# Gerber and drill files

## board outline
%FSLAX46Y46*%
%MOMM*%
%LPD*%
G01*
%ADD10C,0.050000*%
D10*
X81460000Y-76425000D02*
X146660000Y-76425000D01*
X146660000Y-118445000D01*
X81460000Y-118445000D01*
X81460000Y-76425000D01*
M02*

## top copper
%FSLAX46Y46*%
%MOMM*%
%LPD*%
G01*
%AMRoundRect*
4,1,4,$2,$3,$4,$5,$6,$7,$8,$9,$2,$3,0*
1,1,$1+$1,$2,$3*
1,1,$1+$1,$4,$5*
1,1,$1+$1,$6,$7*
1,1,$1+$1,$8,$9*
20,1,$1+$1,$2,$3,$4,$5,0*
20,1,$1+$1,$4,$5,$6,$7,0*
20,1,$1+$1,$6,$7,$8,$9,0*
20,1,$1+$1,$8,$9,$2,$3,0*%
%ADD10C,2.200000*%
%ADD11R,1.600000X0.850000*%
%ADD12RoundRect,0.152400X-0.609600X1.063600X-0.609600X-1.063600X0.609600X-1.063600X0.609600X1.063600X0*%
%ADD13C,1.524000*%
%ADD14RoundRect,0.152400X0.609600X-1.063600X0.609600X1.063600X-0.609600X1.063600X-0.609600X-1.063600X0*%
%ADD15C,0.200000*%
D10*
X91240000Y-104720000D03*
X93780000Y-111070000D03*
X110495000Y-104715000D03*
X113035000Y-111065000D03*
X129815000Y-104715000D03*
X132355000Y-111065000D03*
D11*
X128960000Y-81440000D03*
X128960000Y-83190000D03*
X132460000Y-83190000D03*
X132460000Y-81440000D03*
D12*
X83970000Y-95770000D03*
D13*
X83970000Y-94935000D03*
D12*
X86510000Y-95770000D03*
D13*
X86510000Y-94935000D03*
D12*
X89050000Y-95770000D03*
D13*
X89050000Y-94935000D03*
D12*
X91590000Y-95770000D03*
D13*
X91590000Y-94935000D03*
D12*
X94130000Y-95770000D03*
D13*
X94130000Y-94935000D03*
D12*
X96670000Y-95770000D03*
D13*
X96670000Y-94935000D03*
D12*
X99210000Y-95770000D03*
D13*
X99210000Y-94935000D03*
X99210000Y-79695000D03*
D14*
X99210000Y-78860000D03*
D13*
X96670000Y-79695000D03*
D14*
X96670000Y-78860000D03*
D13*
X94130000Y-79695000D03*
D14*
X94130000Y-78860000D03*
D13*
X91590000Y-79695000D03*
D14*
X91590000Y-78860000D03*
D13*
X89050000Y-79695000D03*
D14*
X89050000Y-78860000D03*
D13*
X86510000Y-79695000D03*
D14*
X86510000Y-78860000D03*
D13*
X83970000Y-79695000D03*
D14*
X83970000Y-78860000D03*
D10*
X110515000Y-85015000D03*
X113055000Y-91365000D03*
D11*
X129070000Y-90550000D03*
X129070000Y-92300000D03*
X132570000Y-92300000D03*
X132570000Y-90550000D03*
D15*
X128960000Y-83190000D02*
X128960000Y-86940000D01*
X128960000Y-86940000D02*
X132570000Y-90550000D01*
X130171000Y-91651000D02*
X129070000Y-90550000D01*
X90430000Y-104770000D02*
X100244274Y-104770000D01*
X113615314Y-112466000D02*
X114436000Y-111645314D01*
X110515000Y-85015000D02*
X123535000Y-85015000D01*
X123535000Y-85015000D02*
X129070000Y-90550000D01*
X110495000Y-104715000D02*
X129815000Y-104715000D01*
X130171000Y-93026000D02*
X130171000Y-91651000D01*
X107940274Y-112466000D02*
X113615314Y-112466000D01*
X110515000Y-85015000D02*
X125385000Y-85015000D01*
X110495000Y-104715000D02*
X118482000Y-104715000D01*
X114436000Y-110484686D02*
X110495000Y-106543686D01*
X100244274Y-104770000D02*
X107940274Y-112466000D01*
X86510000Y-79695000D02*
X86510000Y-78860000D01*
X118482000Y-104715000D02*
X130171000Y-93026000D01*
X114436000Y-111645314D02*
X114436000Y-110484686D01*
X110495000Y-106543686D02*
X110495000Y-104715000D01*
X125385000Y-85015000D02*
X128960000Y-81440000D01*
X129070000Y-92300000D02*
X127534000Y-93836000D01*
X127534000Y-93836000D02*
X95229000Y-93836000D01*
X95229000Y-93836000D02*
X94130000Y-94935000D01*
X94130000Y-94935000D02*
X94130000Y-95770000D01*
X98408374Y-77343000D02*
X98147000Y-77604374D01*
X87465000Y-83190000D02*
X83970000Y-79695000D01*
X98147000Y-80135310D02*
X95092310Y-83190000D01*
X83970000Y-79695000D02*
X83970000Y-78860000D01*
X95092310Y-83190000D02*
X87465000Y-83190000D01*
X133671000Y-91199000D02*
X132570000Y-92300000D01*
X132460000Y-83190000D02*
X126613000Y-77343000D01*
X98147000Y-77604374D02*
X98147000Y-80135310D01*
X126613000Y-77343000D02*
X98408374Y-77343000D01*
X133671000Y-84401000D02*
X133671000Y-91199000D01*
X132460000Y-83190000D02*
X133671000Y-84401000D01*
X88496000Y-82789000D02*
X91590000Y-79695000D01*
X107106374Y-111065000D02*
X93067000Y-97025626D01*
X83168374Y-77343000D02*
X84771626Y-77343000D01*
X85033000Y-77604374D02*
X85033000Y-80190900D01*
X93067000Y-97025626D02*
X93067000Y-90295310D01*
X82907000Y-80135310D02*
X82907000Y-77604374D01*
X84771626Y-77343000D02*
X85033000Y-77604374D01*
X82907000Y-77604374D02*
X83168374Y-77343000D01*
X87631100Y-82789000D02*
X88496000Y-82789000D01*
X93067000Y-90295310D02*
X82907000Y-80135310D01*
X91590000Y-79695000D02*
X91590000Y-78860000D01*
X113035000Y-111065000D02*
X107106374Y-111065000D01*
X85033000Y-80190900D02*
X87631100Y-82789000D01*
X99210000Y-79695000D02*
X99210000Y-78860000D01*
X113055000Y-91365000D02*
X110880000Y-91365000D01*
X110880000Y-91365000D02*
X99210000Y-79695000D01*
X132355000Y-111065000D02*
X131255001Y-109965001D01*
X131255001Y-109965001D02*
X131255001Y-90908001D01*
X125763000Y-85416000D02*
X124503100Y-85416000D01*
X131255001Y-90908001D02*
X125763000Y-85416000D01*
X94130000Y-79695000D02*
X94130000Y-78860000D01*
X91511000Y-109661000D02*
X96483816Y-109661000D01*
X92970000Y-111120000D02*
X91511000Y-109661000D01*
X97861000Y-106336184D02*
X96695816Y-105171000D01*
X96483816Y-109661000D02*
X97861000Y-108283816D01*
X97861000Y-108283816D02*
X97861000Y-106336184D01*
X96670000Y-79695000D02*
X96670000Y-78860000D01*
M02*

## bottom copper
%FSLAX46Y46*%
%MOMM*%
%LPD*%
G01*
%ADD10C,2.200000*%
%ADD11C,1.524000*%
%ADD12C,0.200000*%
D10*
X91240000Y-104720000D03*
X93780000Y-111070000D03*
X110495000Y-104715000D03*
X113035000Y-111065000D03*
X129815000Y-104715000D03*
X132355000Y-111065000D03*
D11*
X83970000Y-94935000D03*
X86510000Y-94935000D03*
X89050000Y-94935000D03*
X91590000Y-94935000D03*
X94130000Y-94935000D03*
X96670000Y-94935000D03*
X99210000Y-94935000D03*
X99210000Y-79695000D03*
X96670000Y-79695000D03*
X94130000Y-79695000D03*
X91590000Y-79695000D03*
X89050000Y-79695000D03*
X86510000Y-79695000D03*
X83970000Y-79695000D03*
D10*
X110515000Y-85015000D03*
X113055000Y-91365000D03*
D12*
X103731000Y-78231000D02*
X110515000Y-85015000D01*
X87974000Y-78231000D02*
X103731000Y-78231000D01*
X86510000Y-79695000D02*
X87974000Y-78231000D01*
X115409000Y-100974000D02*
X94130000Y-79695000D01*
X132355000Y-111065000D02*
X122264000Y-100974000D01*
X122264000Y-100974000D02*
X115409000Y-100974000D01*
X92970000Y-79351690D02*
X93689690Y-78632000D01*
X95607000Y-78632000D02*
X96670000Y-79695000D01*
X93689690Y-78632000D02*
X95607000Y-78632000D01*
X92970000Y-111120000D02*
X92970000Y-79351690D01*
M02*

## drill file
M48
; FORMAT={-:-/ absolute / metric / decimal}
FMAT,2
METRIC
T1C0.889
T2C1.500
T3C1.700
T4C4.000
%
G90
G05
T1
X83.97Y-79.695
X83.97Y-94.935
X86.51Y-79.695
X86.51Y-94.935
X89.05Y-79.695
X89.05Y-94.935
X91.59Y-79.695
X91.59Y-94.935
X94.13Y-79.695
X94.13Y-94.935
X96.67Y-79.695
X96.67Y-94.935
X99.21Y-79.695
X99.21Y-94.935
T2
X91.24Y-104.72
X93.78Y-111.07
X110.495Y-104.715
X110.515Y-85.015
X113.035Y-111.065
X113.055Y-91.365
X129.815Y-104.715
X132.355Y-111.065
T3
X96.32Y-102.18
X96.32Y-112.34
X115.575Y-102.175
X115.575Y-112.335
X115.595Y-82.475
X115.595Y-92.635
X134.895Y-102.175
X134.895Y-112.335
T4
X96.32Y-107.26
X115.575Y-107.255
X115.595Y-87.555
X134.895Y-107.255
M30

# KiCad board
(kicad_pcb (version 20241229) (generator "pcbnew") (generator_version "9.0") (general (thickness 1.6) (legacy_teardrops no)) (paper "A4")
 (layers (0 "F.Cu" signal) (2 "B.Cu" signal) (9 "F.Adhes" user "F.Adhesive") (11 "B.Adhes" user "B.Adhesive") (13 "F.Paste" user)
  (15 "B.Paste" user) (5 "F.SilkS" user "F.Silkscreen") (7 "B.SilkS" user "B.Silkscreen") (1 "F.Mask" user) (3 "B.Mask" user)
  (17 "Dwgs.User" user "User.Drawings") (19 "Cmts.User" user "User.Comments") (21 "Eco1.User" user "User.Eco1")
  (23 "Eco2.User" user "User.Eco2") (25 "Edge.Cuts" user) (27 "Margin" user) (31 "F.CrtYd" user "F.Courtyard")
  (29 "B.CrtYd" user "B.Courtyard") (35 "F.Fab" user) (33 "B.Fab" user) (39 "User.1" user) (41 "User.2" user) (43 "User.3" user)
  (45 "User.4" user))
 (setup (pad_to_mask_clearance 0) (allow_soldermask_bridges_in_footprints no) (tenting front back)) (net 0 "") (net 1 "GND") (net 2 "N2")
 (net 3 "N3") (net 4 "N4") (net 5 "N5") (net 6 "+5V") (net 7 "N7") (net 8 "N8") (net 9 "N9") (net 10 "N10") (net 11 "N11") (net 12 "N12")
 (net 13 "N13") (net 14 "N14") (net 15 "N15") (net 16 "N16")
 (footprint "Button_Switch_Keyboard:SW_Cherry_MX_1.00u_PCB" (layer "F.Cu") (at 91.24 104.72 90)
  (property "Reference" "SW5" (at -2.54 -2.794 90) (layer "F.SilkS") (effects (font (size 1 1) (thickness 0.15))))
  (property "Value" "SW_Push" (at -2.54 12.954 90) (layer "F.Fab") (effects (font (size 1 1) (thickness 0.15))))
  (pad "" np_thru_hole circle (at -7.62 5.08 90) (size 1.7 1.7) (drill 1.7) (layers "*.Cu" "*.Mask"))
  (pad "" np_thru_hole circle (at -2.54 5.08 90) (size 4 4) (drill 4) (layers "*.Cu" "*.Mask"))
  (pad "" np_thru_hole circle (at 2.54 5.08 90) (size 1.7 1.7) (drill 1.7) (layers "*.Cu" "*.Mask"))
  (pad "1" thru_hole circle (at 0 0 90) (size 2.2 2.2) (drill 1.5) (layers "*.Cu" "*.Mask") (remove_unused_layers no) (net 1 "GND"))
  (pad "2" thru_hole circle (at -6.35 2.54 90) (size 2.2 2.2) (drill 1.5) (layers "*.Cu" "*.Mask") (remove_unused_layers no) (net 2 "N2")))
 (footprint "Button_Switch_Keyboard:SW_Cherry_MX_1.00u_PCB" (layer "F.Cu") (at 110.495 104.715 90)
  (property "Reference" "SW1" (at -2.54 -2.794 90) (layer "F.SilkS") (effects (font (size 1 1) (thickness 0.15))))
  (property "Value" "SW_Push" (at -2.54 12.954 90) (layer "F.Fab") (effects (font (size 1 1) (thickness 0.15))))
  (pad "" np_thru_hole circle (at -7.62 5.08 90) (size 1.7 1.7) (drill 1.7) (layers "*.Cu" "*.Mask"))
  (pad "" np_thru_hole circle (at -2.54 5.08 90) (size 4 4) (drill 4) (layers "*.Cu" "*.Mask"))
  (pad "" np_thru_hole circle (at 2.54 5.08 90) (size 1.7 1.7) (drill 1.7) (layers "*.Cu" "*.Mask"))
  (pad "1" thru_hole circle (at 0 0 90) (size 2.2 2.2) (drill 1.5) (layers "*.Cu" "*.Mask") (remove_unused_layers no) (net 1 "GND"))
  (pad "2" thru_hole circle (at -6.35 2.54 90) (size 2.2 2.2) (drill 1.5) (layers "*.Cu" "*.Mask") (remove_unused_layers no) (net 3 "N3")))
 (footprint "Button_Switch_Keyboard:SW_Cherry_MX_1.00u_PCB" (layer "F.Cu") (at 129.815 104.715 90)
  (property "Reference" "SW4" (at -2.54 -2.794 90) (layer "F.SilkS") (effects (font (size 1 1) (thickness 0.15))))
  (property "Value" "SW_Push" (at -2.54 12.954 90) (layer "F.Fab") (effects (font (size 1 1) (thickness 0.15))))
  (pad "" np_thru_hole circle (at -7.62 5.08 90) (size 1.7 1.7) (drill 1.7) (layers "*.Cu" "*.Mask"))
  (pad "" np_thru_hole circle (at -2.54 5.08 90) (size 4 4) (drill 4) (layers "*.Cu" "*.Mask"))
  (pad "" np_thru_hole circle (at 2.54 5.08 90) (size 1.7 1.7) (drill 1.7) (layers "*.Cu" "*.Mask"))
  (pad "1" thru_hole circle (at 0 0 90) (size 2.2 2.2) (drill 1.5) (layers "*.Cu" "*.Mask") (remove_unused_layers no) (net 1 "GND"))
  (pad "2" thru_hole circle (at -6.35 2.54 90) (size 2.2 2.2) (drill 1.5) (layers "*.Cu" "*.Mask") (remove_unused_layers no) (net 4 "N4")))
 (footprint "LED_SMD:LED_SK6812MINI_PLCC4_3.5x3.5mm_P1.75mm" (layer "F.Cu") (at 130.71 82.315)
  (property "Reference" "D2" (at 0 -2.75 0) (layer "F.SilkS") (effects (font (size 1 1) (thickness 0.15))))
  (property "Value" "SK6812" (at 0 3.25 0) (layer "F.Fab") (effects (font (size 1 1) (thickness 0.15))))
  (pad "1" smd rect (at -1.75 -0.875) (size 1.6 0.85) (layers "F.Cu" "F.Mask" "F.Paste") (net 1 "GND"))
  (pad "2" smd rect (at -1.75 0.875) (size 1.6 0.85) (layers "F.Cu" "F.Mask" "F.Paste") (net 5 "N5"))
  (pad "3" smd rect (at 1.75 0.875) (size 1.6 0.85) (layers "F.Cu" "F.Mask" "F.Paste") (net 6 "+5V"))
  (pad "4" smd rect (at 1.75 -0.875) (size 1.6 0.85) (layers "F.Cu" "F.Mask" "F.Paste") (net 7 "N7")))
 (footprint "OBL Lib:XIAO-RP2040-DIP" (layer "F.Cu") (at 91.59 87.315 90)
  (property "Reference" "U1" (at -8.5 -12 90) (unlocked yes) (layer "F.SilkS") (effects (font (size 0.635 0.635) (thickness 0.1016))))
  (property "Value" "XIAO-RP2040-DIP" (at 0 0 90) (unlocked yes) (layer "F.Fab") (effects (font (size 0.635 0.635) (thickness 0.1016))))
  (pad "1" smd roundrect (at -8.455 -7.62 270) (size 2.432 1.524) (layers "F.Cu" "F.Mask") (roundrect_rratio 0.1) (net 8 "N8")
   (thermal_bridge_angle 45))
  (pad "1" thru_hole circle (at -7.62 -7.62 270) (size 1.524 1.524) (drill 0.889) (layers "*.Cu" "*.Mask") (remove_unused_layers no)
   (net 8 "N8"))
  (pad "2" smd roundrect (at -8.455 -5.08 270) (size 2.432 1.524) (layers "F.Cu" "F.Mask") (roundrect_rratio 0.1) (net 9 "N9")
   (thermal_bridge_angle 45))
  (pad "2" thru_hole circle (at -7.62 -5.08 270) (size 1.524 1.524) (drill 0.889) (layers "*.Cu" "*.Mask") (remove_unused_layers no)
   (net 9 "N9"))
  (pad "3" smd roundrect (at -8.455 -2.54 270) (size 2.432 1.524) (layers "F.Cu" "F.Mask") (roundrect_rratio 0.1) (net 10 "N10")
   (thermal_bridge_angle 45))
  (pad "3" thru_hole circle (at -7.62 -2.54 270) (size 1.524 1.524) (drill 0.889) (layers "*.Cu" "*.Mask") (remove_unused_layers no)
   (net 10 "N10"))
  (pad "4" smd roundrect (at -8.455 0 270) (size 2.432 1.524) (layers "F.Cu" "F.Mask") (roundrect_rratio 0.1) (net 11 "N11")
   (thermal_bridge_angle 45))
  (pad "4" thru_hole circle (at -7.62 0 270) (size 1.524 1.524) (drill 0.889) (layers "*.Cu" "*.Mask") (remove_unused_layers no)
   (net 11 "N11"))
  (pad "5" smd roundrect (at -8.455 2.54 270) (size 2.432 1.524) (layers "F.Cu" "F.Mask") (roundrect_rratio 0.1) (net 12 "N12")
   (thermal_bridge_angle 45))
  (pad "5" thru_hole circle (at -7.62 2.54 270) (size 1.524 1.524) (drill 0.889) (layers "*.Cu" "*.Mask") (remove_unused_layers no)
   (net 12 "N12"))
  (pad "6" smd roundrect (at -8.455 5.08 270) (size 2.432 1.524) (layers "F.Cu" "F.Mask") (roundrect_rratio 0.1) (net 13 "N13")
   (thermal_bridge_angle 45))
  (pad "6" thru_hole circle (at -7.62 5.08 270) (size 1.524 1.524) (drill 0.889) (layers "*.Cu" "*.Mask") (remove_unused_layers no)
   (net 13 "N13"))
  (pad "7" smd roundrect (at -8.455 7.62 270) (size 2.432 1.524) (layers "F.Cu" "F.Mask") (roundrect_rratio 0.1) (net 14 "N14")
   (thermal_bridge_angle 45))
  (pad "7" thru_hole circle (at -7.62 7.62 270) (size 1.524 1.524) (drill 0.889) (layers "*.Cu" "*.Mask") (remove_unused_layers no)
   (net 14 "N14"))
  (pad "8" thru_hole circle (at 7.62 7.62 90) (size 1.524 1.524) (drill 0.889) (layers "*.Cu" "*.Mask") (remove_unused_layers no)
   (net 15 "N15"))
  (pad "8" smd roundrect (at 8.455 7.62 90) (size 2.432 1.524) (layers "F.Cu" "F.Mask") (roundrect_rratio 0.1) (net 15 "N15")
   (thermal_bridge_angle 45))
  (pad "9" thru_hole circle (at 7.62 5.08 90) (size 1.524 1.524) (drill 0.889) (layers "*.Cu" "*.Mask") (remove_unused_layers no)
   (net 2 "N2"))
  (pad "9" smd roundrect (at 8.455 5.08 90) (size 2.432 1.524) (layers "F.Cu" "F.Mask") (roundrect_rratio 0.1) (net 2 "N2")
   (thermal_bridge_angle 45))
  (pad "10" thru_hole circle (at 7.62 2.54 90) (size 1.524 1.524) (drill 0.889) (layers "*.Cu" "*.Mask") (remove_unused_layers no)
   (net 4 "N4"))
  (pad "10" smd roundrect (at 8.455 2.54 90) (size 2.432 1.524) (layers "F.Cu" "F.Mask") (roundrect_rratio 0.1) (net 4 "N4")
   (thermal_bridge_angle 45))
  (pad "11" thru_hole circle (at 7.62 0 90) (size 1.524 1.524) (drill 0.889) (layers "*.Cu" "*.Mask") (remove_unused_layers no) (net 3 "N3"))
  (pad "11" smd roundrect (at 8.455 0 90) (size 2.432 1.524) (layers "F.Cu" "F.Mask") (roundrect_rratio 0.1) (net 3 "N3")
   (thermal_bridge_angle 45))
  (pad "12" thru_hole circle (at 7.62 -2.54 90) (size 1.524 1.524) (drill 0.889) (layers "*.Cu" "*.Mask") (remove_unused_layers no)
   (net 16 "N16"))
  (pad "12" smd roundrect (at 8.455 -2.54 90) (size 2.432 1.524) (layers "F.Cu" "F.Mask") (roundrect_rratio 0.1) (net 16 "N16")
   (thermal_bridge_angle 45))
  (pad "13" thru_hole circle (at 7.62 -5.08 90) (size 1.524 1.524) (drill 0.889) (layers "*.Cu" "*.Mask") (remove_unused_layers no)
   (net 1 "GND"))
  (pad "13" smd roundrect (at 8.455 -5.08 90) (size 2.432 1.524) (layers "F.Cu" "F.Mask") (roundrect_rratio 0.1) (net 1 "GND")
   (thermal_bridge_angle 45))
  (pad "14" thru_hole circle (at 7.62 -7.62 90) (size 1.524 1.524) (drill 0.889) (layers "*.Cu" "*.Mask") (remove_unused_layers no)
   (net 6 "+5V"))
  (pad "14" smd roundrect (at 8.455 -7.62 90) (size 2.432 1.524) (layers "F.Cu" "F.Mask") (roundrect_rratio 0.1) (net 6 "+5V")
   (thermal_bridge_angle 45)))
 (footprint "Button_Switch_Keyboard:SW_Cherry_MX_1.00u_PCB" (layer "F.Cu") (at 110.515 85.015 90)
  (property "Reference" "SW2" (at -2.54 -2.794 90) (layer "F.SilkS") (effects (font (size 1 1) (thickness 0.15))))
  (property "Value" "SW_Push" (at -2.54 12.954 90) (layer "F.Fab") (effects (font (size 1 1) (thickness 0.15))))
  (pad "" np_thru_hole circle (at -7.62 5.08 90) (size 1.7 1.7) (drill 1.7) (layers "*.Cu" "*.Mask"))
  (pad "" np_thru_hole circle (at -2.54 5.08 90) (size 4 4) (drill 4) (layers "*.Cu" "*.Mask"))
  (pad "" np_thru_hole circle (at 2.54 5.08 90) (size 1.7 1.7) (drill 1.7) (layers "*.Cu" "*.Mask"))
  (pad "1" thru_hole circle (at 0 0 90) (size 2.2 2.2) (drill 1.5) (layers "*.Cu" "*.Mask") (remove_unused_layers no) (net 1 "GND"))
  (pad "2" thru_hole circle (at -6.35 2.54 90) (size 2.2 2.2) (drill 1.5) (layers "*.Cu" "*.Mask") (remove_unused_layers no) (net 15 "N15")))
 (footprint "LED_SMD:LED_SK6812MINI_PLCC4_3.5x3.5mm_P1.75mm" (layer "F.Cu") (at 130.82 91.425)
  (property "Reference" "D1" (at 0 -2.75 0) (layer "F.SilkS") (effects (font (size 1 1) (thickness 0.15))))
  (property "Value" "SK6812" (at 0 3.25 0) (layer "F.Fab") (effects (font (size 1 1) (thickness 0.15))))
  (pad "1" smd rect (at -1.75 -0.875) (size 1.6 0.85) (layers "F.Cu" "F.Mask" "F.Paste") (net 1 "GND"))
  (pad "2" smd rect (at -1.75 0.875) (size 1.6 0.85) (layers "F.Cu" "F.Mask" "F.Paste") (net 12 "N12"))
  (pad "3" smd rect (at 1.75 0.875) (size 1.6 0.85) (layers "F.Cu" "F.Mask" "F.Paste") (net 6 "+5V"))
  (pad "4" smd rect (at 1.75 -0.875) (size 1.6 0.85) (layers "F.Cu" "F.Mask" "F.Paste") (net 5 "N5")))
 (gr_rect (start 81.46 76.425) (end 146.66 118.445) (stroke (width 0.05) (type default)) (fill no) (layer "Edge.Cuts"))
 (segment (start 128.96 83.19) (end 128.96 86.94) (width 0.2) (layer "F.Cu") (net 5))
 (segment (start 128.96 86.94) (end 132.57 90.55) (width 0.2) (layer "F.Cu") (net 5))
 (segment (start 130.171 91.651) (end 129.07 90.55) (width 0.2) (layer "F.Cu") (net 1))
 (segment (start 90.43 104.77) (end 100.244274 104.77) (width 0.2) (layer "F.Cu") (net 1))
 (segment (start 113.615314 112.466) (end 114.436 111.645314) (width 0.2) (layer "F.Cu") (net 1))
 (segment (start 110.515 85.015) (end 123.535 85.015) (width 0.2) (layer "F.Cu") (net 1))
 (segment (start 123.535 85.015) (end 129.07 90.55) (width 0.2) (layer "F.Cu") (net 1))
 (segment (start 110.495 104.715) (end 129.815 104.715) (width 0.2) (layer "F.Cu") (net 1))
 (segment (start 130.171 93.026) (end 130.171 91.651) (width 0.2) (layer "F.Cu") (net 1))
 (segment (start 107.940274 112.466) (end 113.615314 112.466) (width 0.2) (layer "F.Cu") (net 1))
 (segment (start 110.515 85.015) (end 125.385 85.015) (width 0.2) (layer "F.Cu") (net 1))
 (segment (start 110.495 104.715) (end 118.482 104.715) (width 0.2) (layer "F.Cu") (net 1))
 (segment (start 114.436 110.484686) (end 110.495 106.543686) (width 0.2) (layer "F.Cu") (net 1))
 (segment (start 100.244274 104.77) (end 107.940274 112.466) (width 0.2) (layer "F.Cu") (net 1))
 (segment (start 86.51 79.695) (end 86.51 78.86) (width 0.2) (layer "F.Cu") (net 1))
 (segment (start 118.482 104.715) (end 130.171 93.026) (width 0.2) (layer "F.Cu") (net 1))
 (segment (start 114.436 111.645314) (end 114.436 110.484686) (width 0.2) (layer "F.Cu") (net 1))
 (segment (start 110.495 106.543686) (end 110.495 104.715) (width 0.2) (layer "F.Cu") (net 1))
 (segment (start 125.385 85.015) (end 128.96 81.44) (width 0.2) (layer "F.Cu") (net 1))
 (segment (start 103.731 78.231) (end 110.515 85.015) (width 0.2) (layer "B.Cu") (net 1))
 (segment (start 87.974 78.231) (end 103.731 78.231) (width 0.2) (layer "B.Cu") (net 1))
 (segment (start 86.51 79.695) (end 87.974 78.231) (width 0.2) (layer "B.Cu") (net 1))
 (segment (start 129.07 92.3) (end 127.534 93.836) (width 0.2) (layer "F.Cu") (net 12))
 (segment (start 127.534 93.836) (end 95.229 93.836) (width 0.2) (layer "F.Cu") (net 12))
 (segment (start 95.229 93.836) (end 94.13 94.935) (width 0.2) (layer "F.Cu") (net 12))
 (segment (start 94.13 94.935) (end 94.13 95.77) (width 0.2) (layer "F.Cu") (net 12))
 (segment (start 98.408374 77.343) (end 98.147 77.604374) (width 0.2) (layer "F.Cu") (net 6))
 (segment (start 87.465 83.19) (end 83.97 79.695) (width 0.2) (layer "F.Cu") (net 6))
 (segment (start 98.147 80.13531) (end 95.09231 83.19) (width 0.2) (layer "F.Cu") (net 6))
 (segment (start 83.97 79.695) (end 83.97 78.86) (width 0.2) (layer "F.Cu") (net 6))
 (segment (start 95.09231 83.19) (end 87.465 83.19) (width 0.2) (layer "F.Cu") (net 6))
 (segment (start 133.671 91.199) (end 132.57 92.3) (width 0.2) (layer "F.Cu") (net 6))
 (segment (start 132.46 83.19) (end 126.613 77.343) (width 0.2) (layer "F.Cu") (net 6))
 (segment (start 98.147 77.604374) (end 98.147 80.13531) (width 0.2) (layer "F.Cu") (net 6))
 (segment (start 126.613 77.343) (end 98.408374 77.343) (width 0.2) (layer "F.Cu") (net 6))
 (segment (start 133.671 84.401) (end 133.671 91.199) (width 0.2) (layer "F.Cu") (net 6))
 (segment (start 132.46 83.19) (end 133.671 84.401) (width 0.2) (layer "F.Cu") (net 6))
 (segment (start 88.496 82.789) (end 91.59 79.695) (width 0.2) (layer "F.Cu") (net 3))
 (segment (start 107.106374 111.065) (end 93.067 97.025626) (width 0.2) (layer "F.Cu") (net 3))
 (segment (start 83.168374 77.343) (end 84.771626 77.343) (width 0.2) (layer "F.Cu") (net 3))
 (segment (start 85.033 77.604374) (end 85.033 80.1909) (width 0.2) (layer "F.Cu") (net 3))
 (segment (start 93.067 97.025626) (end 93.067 90.29531) (width 0.2) (layer "F.Cu") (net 3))
 (segment (start 82.907 80.13531) (end 82.907 77.604374) (width 0.2) (layer "F.Cu") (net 3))
 (segment (start 84.771626 77.343) (end 85.033 77.604374) (width 0.2) (layer "F.Cu") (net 3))
 (segment (start 82.907 77.604374) (end 83.168374 77.343) (width 0.2) (layer "F.Cu") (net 3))
 (segment (start 87.6311 82.789) (end 88.496 82.789) (width 0.2) (layer "F.Cu") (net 3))
 (segment (start 93.067 90.29531) (end 82.907 80.13531) (width 0.2) (layer "F.Cu") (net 3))
 (segment (start 91.59 79.695) (end 91.59 78.86) (width 0.2) (layer "F.Cu") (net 3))
 (segment (start 113.035 111.065) (end 107.106374 111.065) (width 0.2) (layer "F.Cu") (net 3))
 (segment (start 85.033 80.1909) (end 87.6311 82.789) (width 0.2) (layer "F.Cu") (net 3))
 (segment (start 99.21 79.695) (end 99.21 78.86) (width 0.2) (layer "F.Cu") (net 15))
 (segment (start 113.055 91.365) (end 110.88 91.365) (width 0.2) (layer "F.Cu") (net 15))
 (segment (start 110.88 91.365) (end 99.21 79.695) (width 0.2) (layer "F.Cu") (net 15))
 (segment (start 132.355 111.065) (end 131.255001 109.965001) (width 0.2) (layer "F.Cu") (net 4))
 (segment (start 131.255001 109.965001) (end 131.255001 90.908001) (width 0.2) (layer "F.Cu") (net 4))
 (segment (start 125.763 85.416) (end 124.5031 85.416) (width 0.2) (layer "F.Cu") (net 4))
 (segment (start 131.255001 90.908001) (end 125.763 85.416) (width 0.2) (layer "F.Cu") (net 4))
 (segment (start 94.13 79.695) (end 94.13 78.86) (width 0.2) (layer "F.Cu") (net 4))
 (segment (start 115.409 100.974) (end 94.13 79.695) (width 0.2) (layer "B.Cu") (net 4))
 (segment (start 132.355 111.065) (end 122.264 100.974) (width 0.2) (layer "B.Cu") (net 4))
 (segment (start 122.264 100.974) (end 115.409 100.974) (width 0.2) (layer "B.Cu") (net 4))
 (segment (start 91.511 109.661) (end 96.483816 109.661) (width 0.2) (layer "F.Cu") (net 2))
 (segment (start 92.97 111.12) (end 91.511 109.661) (width 0.2) (layer "F.Cu") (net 2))
 (segment (start 97.861 106.336184) (end 96.695816 105.171) (width 0.2) (layer "F.Cu") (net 2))
 (segment (start 96.483816 109.661) (end 97.861 108.283816) (width 0.2) (layer "F.Cu") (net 2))
 (segment (start 97.861 108.283816) (end 97.861 106.336184) (width 0.2) (layer "F.Cu") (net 2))
 (segment (start 96.67 79.695) (end 96.67 78.86) (width 0.2) (layer "F.Cu") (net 2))
 (segment (start 92.97 79.35169) (end 93.68969 78.632) (width 0.2) (layer "B.Cu") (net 2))
 (segment (start 95.607 78.632) (end 96.67 79.695) (width 0.2) (layer "B.Cu") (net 2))
 (segment (start 93.68969 78.632) (end 95.607 78.632) (width 0.2) (layer "B.Cu") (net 2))
 (segment (start 92.97 111.12) (end 92.97 79.35169) (width 0.2) (layer "B.Cu") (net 2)))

